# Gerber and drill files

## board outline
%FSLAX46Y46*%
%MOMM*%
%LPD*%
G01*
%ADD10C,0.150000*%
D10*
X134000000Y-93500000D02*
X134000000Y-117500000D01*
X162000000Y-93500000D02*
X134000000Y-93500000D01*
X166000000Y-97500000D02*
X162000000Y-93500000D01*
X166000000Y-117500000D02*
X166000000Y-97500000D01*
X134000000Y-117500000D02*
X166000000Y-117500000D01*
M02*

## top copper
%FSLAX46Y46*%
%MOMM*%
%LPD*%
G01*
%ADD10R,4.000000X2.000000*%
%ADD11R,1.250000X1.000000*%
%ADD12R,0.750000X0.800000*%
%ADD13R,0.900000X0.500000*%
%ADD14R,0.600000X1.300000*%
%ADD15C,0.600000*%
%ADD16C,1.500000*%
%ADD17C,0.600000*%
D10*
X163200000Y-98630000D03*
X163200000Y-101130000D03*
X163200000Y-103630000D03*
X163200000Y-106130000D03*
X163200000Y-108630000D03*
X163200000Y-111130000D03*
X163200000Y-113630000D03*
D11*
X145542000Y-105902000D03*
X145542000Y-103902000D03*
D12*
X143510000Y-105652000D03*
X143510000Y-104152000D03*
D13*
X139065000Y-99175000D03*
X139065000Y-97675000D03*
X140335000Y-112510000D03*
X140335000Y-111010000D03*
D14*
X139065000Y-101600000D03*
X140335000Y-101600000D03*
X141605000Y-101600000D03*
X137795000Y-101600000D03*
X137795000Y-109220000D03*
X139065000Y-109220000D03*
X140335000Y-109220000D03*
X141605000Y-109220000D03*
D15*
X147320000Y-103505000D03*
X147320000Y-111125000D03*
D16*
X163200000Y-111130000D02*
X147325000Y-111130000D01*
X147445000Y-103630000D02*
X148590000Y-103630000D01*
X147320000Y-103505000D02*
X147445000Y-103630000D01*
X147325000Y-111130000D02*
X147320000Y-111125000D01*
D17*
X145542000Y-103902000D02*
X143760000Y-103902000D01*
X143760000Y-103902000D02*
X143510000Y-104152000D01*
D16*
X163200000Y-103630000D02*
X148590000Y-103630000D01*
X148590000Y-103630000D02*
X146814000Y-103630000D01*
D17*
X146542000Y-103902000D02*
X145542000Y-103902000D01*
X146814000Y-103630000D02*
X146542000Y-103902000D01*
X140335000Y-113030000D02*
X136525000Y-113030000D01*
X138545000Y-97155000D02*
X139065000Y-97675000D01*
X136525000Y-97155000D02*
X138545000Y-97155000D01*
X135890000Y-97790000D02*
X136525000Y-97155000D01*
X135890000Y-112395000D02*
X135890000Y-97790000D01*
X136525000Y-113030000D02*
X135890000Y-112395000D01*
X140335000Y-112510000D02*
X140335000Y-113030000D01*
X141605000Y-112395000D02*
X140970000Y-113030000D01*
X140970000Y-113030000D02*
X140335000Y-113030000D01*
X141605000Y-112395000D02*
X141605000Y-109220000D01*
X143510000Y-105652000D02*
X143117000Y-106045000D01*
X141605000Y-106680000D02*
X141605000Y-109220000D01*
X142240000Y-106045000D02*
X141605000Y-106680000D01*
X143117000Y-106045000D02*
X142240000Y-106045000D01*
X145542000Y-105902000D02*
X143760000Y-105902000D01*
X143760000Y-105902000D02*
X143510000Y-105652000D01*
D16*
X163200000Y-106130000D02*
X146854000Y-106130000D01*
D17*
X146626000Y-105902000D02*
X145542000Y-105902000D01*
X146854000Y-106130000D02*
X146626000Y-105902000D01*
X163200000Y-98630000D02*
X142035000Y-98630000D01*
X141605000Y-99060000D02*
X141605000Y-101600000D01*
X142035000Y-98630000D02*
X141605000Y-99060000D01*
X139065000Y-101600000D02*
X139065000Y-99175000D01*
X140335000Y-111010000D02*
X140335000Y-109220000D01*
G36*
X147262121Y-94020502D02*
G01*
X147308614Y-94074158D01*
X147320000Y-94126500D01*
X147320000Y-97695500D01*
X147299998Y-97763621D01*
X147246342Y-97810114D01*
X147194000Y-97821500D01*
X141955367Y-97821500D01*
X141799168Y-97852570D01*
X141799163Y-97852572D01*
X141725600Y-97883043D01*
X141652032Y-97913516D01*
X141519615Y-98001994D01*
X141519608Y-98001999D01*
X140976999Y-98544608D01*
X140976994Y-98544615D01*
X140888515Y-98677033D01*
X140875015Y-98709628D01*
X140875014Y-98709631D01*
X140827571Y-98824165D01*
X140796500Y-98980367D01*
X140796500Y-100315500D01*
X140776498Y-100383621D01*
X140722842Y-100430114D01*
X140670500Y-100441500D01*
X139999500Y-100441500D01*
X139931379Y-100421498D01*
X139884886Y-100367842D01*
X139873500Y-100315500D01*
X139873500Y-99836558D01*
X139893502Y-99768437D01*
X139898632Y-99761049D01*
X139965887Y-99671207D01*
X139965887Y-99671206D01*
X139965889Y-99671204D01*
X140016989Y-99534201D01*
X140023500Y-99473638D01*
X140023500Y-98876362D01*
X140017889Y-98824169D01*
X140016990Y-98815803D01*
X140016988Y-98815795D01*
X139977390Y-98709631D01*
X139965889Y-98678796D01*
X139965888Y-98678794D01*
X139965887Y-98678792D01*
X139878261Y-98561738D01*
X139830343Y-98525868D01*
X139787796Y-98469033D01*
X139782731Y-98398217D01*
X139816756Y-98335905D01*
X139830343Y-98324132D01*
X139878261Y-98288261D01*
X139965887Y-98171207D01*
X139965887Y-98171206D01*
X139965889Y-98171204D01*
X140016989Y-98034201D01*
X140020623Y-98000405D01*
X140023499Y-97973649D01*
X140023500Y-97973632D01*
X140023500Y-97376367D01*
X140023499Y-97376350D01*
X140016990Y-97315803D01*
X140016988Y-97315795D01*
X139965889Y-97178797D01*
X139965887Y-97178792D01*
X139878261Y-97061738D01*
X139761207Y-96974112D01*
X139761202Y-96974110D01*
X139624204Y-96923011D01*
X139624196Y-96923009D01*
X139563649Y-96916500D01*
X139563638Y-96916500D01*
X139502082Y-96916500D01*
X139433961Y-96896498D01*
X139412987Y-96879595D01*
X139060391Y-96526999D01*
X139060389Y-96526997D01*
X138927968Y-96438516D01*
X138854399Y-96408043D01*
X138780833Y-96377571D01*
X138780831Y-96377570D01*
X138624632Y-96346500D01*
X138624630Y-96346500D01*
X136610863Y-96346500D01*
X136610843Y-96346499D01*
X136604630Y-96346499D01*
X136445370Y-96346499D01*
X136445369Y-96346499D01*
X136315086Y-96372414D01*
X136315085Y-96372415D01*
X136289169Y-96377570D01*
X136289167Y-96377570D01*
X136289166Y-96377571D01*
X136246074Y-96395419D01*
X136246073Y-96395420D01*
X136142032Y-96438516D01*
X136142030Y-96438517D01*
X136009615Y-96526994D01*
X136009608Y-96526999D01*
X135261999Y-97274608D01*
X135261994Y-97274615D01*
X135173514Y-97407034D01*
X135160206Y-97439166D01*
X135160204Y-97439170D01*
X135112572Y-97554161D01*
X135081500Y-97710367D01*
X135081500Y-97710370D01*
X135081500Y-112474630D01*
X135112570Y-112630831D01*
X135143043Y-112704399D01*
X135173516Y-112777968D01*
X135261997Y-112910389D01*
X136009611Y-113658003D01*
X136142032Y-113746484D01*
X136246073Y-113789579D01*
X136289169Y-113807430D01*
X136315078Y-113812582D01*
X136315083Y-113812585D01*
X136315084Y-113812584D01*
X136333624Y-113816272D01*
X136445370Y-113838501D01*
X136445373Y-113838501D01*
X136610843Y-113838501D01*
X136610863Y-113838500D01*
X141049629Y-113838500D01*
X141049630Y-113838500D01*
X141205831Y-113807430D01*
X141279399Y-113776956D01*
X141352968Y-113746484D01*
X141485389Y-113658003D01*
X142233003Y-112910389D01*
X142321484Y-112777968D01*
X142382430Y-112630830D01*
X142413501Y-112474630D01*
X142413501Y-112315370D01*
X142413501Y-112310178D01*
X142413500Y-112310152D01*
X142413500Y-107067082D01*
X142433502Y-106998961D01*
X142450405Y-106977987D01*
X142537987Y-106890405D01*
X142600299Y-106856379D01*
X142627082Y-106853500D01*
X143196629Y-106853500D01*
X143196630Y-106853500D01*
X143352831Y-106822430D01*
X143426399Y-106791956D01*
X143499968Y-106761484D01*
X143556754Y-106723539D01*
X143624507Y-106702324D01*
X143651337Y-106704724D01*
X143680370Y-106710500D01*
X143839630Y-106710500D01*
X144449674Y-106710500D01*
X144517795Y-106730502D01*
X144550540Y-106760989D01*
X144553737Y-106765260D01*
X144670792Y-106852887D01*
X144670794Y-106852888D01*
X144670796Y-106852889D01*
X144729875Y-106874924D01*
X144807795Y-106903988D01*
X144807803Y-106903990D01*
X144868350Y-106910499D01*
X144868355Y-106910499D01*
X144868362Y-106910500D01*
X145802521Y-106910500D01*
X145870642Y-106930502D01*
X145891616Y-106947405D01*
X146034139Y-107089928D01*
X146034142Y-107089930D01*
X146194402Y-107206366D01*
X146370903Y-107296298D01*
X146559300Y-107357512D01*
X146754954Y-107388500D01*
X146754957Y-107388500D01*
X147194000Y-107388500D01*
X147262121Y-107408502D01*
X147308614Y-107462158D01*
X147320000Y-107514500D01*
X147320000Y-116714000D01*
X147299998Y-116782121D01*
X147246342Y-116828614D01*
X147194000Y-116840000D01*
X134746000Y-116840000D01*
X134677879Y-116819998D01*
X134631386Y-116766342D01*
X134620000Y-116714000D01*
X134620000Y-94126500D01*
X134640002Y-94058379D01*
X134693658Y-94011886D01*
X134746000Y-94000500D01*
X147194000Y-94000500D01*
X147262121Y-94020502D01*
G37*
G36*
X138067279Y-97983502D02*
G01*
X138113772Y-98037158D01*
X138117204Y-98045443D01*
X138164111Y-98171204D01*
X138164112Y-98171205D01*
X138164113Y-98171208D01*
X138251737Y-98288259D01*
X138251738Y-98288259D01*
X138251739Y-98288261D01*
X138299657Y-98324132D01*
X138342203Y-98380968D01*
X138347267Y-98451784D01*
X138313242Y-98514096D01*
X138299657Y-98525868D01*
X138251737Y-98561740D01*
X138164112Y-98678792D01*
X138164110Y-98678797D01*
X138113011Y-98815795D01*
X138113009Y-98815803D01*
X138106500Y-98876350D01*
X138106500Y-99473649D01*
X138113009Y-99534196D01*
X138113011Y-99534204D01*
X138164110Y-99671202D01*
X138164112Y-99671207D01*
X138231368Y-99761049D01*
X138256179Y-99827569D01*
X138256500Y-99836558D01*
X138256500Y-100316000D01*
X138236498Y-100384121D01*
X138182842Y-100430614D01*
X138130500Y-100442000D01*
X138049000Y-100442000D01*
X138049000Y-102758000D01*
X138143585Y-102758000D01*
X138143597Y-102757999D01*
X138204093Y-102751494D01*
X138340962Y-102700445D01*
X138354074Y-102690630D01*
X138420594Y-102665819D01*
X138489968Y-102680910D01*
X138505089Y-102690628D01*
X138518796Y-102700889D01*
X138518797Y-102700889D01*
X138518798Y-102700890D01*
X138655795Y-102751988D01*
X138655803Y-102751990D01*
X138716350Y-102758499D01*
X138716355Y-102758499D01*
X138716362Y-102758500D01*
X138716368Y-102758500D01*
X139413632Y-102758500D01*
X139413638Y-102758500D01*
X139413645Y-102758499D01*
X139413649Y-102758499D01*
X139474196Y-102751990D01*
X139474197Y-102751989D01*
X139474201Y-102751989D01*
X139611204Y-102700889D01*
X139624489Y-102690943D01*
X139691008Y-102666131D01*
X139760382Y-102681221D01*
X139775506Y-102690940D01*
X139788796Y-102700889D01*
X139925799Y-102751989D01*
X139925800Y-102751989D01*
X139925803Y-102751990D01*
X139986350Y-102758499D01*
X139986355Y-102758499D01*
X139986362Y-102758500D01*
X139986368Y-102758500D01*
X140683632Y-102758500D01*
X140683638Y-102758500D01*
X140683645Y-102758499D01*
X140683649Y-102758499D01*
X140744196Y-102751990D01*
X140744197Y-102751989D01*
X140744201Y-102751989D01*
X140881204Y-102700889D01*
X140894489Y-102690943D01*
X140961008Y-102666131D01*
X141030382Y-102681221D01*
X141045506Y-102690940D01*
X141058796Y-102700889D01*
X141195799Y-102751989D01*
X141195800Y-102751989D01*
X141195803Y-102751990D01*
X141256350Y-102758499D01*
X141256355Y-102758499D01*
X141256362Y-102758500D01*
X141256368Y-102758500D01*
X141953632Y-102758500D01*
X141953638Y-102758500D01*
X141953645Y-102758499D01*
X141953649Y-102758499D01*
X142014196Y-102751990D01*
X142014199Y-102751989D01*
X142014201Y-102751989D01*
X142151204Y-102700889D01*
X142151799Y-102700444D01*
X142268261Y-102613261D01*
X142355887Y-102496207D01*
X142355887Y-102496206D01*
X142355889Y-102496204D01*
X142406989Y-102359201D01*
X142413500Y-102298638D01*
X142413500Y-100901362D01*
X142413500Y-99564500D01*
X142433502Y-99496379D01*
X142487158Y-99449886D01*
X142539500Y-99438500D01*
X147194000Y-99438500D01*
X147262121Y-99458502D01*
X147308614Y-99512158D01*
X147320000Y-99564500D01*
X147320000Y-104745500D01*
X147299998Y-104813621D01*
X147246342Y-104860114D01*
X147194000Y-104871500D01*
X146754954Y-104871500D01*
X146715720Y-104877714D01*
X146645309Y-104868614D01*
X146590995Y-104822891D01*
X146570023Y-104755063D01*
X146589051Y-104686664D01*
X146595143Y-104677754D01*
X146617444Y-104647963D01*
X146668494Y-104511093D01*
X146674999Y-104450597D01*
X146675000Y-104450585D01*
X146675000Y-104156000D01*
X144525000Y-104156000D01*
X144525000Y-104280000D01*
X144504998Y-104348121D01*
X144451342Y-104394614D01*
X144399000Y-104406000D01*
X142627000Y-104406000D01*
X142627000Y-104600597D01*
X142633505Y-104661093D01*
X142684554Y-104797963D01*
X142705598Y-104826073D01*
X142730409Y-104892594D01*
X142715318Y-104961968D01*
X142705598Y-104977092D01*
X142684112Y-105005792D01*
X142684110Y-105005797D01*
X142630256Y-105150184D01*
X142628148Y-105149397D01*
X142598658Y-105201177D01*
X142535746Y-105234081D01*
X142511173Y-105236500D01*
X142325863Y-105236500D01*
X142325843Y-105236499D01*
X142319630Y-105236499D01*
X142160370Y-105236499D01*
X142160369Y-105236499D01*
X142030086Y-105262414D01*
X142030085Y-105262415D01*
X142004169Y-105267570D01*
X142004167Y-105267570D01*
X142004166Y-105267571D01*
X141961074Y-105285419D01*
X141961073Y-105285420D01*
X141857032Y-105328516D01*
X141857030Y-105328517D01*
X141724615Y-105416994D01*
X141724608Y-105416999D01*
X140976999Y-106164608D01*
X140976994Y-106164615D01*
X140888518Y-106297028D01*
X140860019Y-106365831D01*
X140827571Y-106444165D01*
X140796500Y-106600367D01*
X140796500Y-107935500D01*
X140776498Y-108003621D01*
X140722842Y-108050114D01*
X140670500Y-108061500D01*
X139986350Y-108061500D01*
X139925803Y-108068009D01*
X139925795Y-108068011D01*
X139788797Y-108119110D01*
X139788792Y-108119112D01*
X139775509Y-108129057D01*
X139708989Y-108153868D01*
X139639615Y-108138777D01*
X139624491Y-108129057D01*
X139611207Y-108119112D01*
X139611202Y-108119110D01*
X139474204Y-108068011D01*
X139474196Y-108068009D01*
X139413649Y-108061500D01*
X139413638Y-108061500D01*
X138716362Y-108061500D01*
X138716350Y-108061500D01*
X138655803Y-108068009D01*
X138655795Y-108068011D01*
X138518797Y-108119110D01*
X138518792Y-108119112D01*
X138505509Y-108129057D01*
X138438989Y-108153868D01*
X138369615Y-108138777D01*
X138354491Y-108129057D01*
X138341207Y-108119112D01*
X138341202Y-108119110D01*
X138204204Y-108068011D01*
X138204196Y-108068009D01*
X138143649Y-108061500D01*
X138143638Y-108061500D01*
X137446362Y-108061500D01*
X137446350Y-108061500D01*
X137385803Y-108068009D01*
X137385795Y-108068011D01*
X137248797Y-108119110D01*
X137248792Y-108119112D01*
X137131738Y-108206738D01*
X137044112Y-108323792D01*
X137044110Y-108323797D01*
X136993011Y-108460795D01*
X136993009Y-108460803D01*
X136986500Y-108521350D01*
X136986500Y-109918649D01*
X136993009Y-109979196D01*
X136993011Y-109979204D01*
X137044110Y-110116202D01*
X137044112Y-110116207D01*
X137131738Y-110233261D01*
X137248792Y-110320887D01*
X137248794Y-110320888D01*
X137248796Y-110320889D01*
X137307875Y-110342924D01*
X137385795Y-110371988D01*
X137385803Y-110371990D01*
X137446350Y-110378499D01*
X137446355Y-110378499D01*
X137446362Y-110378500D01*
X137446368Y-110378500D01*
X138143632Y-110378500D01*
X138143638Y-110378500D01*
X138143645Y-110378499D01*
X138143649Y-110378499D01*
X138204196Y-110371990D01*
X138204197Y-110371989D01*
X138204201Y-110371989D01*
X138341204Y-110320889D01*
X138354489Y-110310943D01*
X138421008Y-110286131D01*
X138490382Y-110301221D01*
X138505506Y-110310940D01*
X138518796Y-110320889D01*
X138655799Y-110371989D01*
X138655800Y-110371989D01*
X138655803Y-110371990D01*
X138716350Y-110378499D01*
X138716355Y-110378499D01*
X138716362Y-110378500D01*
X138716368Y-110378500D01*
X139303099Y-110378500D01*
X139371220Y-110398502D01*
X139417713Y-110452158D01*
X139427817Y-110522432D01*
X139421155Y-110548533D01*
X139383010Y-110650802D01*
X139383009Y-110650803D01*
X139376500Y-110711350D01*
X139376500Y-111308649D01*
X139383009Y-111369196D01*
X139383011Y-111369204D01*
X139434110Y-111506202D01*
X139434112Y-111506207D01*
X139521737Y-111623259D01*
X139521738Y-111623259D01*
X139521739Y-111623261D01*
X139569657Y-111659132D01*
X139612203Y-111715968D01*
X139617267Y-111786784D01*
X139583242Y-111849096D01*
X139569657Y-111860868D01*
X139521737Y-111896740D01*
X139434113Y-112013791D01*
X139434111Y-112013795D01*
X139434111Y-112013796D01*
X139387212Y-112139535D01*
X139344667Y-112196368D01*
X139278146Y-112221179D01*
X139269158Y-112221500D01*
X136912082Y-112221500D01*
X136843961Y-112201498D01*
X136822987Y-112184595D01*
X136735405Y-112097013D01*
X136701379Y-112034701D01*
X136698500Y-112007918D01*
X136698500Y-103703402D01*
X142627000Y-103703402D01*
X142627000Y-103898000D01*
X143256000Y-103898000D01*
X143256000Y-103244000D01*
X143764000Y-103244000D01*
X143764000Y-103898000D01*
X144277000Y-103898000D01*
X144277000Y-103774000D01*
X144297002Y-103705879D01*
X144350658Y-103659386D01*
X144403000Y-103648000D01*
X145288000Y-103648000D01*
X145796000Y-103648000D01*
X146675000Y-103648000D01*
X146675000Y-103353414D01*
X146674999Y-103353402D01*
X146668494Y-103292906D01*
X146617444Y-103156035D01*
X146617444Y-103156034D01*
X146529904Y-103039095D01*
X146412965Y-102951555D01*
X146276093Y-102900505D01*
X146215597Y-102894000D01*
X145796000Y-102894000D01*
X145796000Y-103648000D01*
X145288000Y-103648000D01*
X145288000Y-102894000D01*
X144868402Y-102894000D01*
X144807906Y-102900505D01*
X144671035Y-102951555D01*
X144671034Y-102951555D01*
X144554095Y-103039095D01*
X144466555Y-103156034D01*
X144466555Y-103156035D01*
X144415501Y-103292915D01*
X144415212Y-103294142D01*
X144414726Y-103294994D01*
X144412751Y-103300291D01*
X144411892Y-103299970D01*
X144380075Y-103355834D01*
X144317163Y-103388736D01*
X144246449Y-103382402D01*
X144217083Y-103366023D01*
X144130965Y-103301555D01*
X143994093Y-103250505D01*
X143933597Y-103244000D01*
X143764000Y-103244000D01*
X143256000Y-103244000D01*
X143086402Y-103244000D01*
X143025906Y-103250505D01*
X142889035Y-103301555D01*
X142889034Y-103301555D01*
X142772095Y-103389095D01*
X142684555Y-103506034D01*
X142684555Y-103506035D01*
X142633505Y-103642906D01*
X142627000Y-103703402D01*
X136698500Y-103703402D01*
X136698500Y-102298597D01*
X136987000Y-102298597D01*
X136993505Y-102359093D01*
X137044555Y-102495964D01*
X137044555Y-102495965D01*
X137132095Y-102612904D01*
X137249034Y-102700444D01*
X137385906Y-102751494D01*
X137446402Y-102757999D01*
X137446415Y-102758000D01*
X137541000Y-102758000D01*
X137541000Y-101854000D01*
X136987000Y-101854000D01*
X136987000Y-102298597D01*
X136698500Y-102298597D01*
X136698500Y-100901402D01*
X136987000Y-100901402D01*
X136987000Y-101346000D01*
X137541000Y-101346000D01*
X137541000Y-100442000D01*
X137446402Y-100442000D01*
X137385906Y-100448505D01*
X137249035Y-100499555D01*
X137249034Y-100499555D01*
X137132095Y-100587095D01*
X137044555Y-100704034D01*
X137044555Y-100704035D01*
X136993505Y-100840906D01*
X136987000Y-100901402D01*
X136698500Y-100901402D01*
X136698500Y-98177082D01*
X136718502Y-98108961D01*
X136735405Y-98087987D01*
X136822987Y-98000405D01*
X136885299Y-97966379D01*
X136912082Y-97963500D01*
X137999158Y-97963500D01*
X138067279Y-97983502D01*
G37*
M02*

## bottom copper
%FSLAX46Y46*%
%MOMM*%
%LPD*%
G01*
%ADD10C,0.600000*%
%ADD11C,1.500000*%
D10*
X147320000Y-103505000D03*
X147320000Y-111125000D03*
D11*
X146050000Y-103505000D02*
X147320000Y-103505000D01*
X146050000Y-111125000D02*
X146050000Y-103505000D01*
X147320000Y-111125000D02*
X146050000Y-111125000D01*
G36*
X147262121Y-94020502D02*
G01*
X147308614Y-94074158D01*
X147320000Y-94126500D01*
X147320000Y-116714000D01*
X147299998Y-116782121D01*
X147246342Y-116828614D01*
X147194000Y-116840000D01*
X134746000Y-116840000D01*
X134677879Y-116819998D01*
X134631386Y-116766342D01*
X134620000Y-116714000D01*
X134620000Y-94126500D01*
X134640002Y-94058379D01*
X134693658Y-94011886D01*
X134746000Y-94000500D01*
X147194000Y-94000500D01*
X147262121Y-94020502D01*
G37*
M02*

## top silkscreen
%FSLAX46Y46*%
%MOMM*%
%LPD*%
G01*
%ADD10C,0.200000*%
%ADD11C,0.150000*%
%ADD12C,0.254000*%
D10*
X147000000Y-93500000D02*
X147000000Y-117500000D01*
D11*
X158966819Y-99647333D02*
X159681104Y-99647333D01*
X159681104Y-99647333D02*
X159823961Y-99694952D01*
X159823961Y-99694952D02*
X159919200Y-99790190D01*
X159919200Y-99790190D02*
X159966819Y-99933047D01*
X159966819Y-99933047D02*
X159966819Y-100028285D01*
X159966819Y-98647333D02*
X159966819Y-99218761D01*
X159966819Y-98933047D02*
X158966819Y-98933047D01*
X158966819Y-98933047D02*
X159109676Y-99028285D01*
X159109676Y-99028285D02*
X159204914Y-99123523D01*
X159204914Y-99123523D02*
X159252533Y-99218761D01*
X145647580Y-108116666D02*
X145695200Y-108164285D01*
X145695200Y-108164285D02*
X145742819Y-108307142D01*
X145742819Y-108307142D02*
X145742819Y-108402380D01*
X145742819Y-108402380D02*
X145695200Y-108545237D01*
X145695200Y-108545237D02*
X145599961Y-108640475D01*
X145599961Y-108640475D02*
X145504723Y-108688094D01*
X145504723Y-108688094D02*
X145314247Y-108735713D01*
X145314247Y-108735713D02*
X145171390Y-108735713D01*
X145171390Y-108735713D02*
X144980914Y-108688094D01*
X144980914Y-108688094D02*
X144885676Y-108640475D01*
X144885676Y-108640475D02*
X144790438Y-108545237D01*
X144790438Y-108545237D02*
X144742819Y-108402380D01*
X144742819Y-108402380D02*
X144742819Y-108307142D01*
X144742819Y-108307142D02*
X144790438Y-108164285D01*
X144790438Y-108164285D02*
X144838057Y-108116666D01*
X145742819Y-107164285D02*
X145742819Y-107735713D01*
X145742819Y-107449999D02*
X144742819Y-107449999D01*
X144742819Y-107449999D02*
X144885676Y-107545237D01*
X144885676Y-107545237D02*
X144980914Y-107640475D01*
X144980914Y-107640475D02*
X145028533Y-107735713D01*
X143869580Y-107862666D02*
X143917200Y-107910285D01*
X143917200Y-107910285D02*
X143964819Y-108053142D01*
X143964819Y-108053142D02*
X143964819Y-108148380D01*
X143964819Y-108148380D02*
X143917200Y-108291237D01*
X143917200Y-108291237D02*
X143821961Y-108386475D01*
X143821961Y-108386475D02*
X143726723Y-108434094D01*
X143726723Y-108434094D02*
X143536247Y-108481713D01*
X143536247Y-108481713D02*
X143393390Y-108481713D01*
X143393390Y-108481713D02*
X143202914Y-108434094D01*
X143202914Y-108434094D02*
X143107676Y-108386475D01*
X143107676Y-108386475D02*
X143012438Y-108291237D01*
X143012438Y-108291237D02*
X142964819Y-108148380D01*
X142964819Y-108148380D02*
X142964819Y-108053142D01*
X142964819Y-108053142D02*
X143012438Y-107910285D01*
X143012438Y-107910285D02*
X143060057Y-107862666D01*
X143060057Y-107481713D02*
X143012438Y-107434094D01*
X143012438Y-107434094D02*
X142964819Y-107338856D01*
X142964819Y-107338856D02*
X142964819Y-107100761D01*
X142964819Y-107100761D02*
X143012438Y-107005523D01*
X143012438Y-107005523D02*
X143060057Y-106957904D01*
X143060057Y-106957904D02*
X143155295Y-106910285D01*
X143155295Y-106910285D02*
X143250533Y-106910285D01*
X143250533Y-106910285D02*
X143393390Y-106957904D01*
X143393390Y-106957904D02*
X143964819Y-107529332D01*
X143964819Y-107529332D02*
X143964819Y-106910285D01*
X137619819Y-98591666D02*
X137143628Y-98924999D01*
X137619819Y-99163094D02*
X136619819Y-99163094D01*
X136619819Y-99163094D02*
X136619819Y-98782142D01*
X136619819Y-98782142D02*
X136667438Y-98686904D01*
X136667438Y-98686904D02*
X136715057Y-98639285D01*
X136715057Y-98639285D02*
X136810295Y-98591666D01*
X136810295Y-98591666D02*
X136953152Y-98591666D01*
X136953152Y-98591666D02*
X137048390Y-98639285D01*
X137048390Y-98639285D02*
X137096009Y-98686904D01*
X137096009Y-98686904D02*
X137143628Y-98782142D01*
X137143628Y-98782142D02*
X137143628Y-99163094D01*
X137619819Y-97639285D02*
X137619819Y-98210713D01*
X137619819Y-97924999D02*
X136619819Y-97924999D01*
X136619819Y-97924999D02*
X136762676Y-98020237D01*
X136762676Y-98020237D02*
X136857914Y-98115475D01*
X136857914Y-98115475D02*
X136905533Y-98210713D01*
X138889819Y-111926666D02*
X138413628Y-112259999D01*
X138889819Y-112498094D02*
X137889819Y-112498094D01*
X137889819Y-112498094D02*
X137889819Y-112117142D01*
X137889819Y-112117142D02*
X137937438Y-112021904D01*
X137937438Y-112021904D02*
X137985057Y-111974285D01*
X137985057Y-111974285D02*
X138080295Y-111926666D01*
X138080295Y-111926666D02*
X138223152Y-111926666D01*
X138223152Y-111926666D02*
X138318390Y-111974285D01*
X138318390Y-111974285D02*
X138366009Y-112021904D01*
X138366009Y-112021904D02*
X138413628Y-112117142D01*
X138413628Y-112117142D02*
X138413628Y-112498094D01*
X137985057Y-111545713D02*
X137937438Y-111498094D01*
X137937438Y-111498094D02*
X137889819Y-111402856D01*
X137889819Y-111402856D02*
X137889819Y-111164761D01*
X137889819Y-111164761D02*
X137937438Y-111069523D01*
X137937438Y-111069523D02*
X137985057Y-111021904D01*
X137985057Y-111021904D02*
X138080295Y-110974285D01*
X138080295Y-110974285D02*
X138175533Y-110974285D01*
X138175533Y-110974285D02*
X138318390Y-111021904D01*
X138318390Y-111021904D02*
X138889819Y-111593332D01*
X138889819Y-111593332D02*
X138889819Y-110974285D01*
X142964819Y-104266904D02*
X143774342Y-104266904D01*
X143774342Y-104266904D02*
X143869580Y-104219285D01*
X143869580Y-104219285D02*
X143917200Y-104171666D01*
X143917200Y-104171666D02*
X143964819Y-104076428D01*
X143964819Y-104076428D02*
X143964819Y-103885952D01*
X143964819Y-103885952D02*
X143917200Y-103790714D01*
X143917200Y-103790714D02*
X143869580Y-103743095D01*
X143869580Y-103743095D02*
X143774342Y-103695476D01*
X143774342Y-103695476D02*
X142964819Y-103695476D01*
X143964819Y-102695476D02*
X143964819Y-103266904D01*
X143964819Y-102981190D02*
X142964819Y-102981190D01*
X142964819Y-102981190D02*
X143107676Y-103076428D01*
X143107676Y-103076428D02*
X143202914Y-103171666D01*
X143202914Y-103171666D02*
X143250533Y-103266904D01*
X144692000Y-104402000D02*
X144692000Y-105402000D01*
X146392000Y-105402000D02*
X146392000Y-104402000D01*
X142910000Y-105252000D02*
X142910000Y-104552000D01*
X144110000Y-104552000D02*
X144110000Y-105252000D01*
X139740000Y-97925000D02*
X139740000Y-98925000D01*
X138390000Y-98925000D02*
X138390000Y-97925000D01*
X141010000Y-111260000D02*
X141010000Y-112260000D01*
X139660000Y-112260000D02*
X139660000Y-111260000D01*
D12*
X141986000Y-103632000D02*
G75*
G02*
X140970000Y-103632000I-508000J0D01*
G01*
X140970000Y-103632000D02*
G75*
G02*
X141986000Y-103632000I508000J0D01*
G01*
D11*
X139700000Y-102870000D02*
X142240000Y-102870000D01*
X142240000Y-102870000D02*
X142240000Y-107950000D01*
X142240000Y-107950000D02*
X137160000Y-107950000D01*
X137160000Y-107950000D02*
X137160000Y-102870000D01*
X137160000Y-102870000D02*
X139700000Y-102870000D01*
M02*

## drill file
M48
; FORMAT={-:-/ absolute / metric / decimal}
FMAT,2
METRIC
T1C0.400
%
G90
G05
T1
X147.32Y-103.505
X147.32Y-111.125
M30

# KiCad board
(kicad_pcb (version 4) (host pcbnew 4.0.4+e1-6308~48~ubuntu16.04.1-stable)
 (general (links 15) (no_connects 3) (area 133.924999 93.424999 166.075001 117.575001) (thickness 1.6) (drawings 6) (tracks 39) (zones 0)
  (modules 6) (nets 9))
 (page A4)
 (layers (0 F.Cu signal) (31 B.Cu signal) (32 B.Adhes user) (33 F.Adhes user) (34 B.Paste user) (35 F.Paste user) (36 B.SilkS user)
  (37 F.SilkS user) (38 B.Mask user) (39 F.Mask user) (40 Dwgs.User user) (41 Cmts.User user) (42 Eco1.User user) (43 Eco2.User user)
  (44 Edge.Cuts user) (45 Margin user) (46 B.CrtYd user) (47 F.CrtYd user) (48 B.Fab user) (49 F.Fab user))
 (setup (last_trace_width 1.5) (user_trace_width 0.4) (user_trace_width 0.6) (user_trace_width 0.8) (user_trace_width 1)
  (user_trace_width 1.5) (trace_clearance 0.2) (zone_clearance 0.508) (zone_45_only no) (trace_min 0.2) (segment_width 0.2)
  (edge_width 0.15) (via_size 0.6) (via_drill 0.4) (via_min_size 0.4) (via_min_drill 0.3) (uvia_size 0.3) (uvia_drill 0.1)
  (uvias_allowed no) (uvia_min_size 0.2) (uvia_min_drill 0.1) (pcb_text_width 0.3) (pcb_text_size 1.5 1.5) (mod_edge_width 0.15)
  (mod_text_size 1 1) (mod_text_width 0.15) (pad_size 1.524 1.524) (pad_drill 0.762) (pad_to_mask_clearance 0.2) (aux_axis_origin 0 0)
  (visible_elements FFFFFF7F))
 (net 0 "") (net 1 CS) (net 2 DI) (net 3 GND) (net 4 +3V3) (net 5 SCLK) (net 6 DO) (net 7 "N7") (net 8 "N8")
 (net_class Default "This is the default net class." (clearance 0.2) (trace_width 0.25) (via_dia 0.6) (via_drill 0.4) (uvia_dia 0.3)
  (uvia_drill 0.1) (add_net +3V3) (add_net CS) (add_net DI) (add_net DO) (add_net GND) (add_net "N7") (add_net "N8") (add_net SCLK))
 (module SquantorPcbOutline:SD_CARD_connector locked (layer F.Cu) (at 163.2 106.13)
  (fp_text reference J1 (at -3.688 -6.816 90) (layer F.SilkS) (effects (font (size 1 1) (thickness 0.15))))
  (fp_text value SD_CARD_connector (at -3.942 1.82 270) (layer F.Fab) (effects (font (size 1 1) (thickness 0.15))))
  (pad 1 smd rect (at 0 -7.5 90) (size 2 4) (layers F.Cu F.Paste F.Mask) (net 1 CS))
  (pad 2 smd rect (at 0 -5 90) (size 2 4) (layers F.Cu F.Paste F.Mask) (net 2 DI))
  (pad 3 smd rect (at 0 -2.5 90) (size 2 4) (layers F.Cu F.Paste F.Mask) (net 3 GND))
  (pad 4 smd rect (at 0 0 90) (size 2 4) (layers F.Cu F.Paste F.Mask) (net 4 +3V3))
  (pad 5 smd rect (at 0 2.5 90) (size 2 4) (layers F.Cu F.Paste F.Mask) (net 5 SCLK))
  (pad 6 smd rect (at 0 5 90) (size 2 4) (layers F.Cu F.Paste F.Mask) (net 3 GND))
  (pad 7 smd rect (at 0 7.5 90) (size 2 4) (layers F.Cu F.Paste F.Mask) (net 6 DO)))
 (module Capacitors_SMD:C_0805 (layer F.Cu) (at 145.542 104.902 90)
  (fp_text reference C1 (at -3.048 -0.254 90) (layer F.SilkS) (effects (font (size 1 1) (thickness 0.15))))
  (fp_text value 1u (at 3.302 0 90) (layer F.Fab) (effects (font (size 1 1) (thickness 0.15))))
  (fp_line (start 0.5 -0.85) (end -0.5 -0.85) (layer F.SilkS) (width 0.15))
  (fp_line (start -0.5 0.85) (end 0.5 0.85) (layer F.SilkS) (width 0.15))
  (pad 1 smd rect (at -1 0 90) (size 1 1.25) (layers F.Cu F.Paste F.Mask) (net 4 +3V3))
  (pad 2 smd rect (at 1 0 90) (size 1 1.25) (layers F.Cu F.Paste F.Mask) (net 3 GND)))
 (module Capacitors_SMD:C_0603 (layer F.Cu) (at 143.51 104.902 90)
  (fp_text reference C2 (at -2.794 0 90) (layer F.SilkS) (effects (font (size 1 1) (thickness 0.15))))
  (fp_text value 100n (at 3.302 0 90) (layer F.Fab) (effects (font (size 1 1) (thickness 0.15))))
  (fp_line (start -0.35 -0.6) (end 0.35 -0.6) (layer F.SilkS) (width 0.15))
  (fp_line (start 0.35 0.6) (end -0.35 0.6) (layer F.SilkS) (width 0.15))
  (pad 1 smd rect (at -0.75 0 90) (size 0.8 0.75) (layers F.Cu F.Paste F.Mask) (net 4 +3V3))
  (pad 2 smd rect (at 0.75 0 90) (size 0.8 0.75) (layers F.Cu F.Paste F.Mask) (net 3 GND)))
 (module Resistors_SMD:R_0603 (layer F.Cu) (at 139.065 98.425 90)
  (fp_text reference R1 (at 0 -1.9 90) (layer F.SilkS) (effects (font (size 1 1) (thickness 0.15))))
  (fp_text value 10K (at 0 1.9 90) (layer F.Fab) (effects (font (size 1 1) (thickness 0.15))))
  (fp_line (start 0.5 0.675) (end -0.5 0.675) (layer F.SilkS) (width 0.15))
  (fp_line (start -0.5 -0.675) (end 0.5 -0.675) (layer F.SilkS) (width 0.15))
  (pad 1 smd rect (at -0.75 0 90) (size 0.5 0.9) (layers F.Cu F.Paste F.Mask) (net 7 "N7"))
  (pad 2 smd rect (at 0.75 0 90) (size 0.5 0.9) (layers F.Cu F.Paste F.Mask) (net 4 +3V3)))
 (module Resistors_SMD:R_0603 (layer F.Cu) (at 140.335 111.76 90)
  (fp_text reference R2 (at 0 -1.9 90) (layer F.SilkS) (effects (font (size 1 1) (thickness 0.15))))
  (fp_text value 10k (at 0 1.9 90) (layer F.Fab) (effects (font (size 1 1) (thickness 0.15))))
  (fp_line (start 0.5 0.675) (end -0.5 0.675) (layer F.SilkS) (width 0.15))
  (fp_line (start -0.5 -0.675) (end 0.5 -0.675) (layer F.SilkS) (width 0.15))
  (pad 1 smd rect (at -0.75 0 90) (size 0.5 0.9) (layers F.Cu F.Paste F.Mask) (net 4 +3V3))
  (pad 2 smd rect (at 0.75 0 90) (size 0.5 0.9) (layers F.Cu F.Paste F.Mask) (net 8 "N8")))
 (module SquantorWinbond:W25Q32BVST (layer F.Cu) (at 139.7 105.41 270)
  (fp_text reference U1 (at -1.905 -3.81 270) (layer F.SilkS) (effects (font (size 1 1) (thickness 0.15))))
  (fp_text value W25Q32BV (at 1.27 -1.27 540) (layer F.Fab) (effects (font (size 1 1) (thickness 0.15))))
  (fp_circle (center -1.778 -1.778) (end -1.27 -1.778) (layer F.SilkS) (width 0.254))
  (fp_line (start -2.54 0) (end -2.54 -2.54) (layer F.SilkS) (width 0.15))
  (fp_line (start -2.54 -2.54) (end 2.54 -2.54) (layer F.SilkS) (width 0.15))
  (fp_line (start 2.54 -2.54) (end 2.54 2.54) (layer F.SilkS) (width 0.15))
  (fp_line (start 2.54 2.54) (end -2.54 2.54) (layer F.SilkS) (width 0.15))
  (fp_line (start -2.54 2.54) (end -2.54 0) (layer F.SilkS) (width 0.15))
  (pad 3 smd rect (at -3.81 0.635 270) (size 1.3 0.6) (layers F.Cu F.Paste F.Mask) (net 7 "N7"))
  (pad 2 smd rect (at -3.81 -0.635 270) (size 1.3 0.6) (layers F.Cu F.Paste F.Mask) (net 6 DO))
  (pad 1 smd rect (at -3.81 -1.905 270) (size 1.3 0.6) (layers F.Cu F.Paste F.Mask) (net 1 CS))
  (pad 4 smd rect (at -3.81 1.905 270) (size 1.3 0.6) (layers F.Cu F.Paste F.Mask) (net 3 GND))
  (pad 5 smd rect (at 3.81 1.905 270) (size 1.3 0.6) (layers F.Cu F.Paste F.Mask) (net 2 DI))
  (pad 6 smd rect (at 3.81 0.635 270) (size 1.3 0.6) (layers F.Cu F.Paste F.Mask) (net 5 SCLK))
  (pad 7 smd rect (at 3.81 -0.635 270) (size 1.3 0.6) (layers F.Cu F.Paste F.Mask) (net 8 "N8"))
  (pad 8 smd rect (at 3.81 -1.905 270) (size 1.3 0.6) (layers F.Cu F.Paste F.Mask) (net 4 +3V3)))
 (gr_line (start 147 93.5) (end 147 117.5) (angle 90) (layer F.SilkS) (width 0.2))
 (gr_line (start 134 93.5) (end 134 117.5) (angle 90) (layer Edge.Cuts) (width 0.15))
 (gr_line (start 162 93.5) (end 134 93.5) (angle 90) (layer Edge.Cuts) (width 0.15))
 (gr_line (start 166 97.5) (end 162 93.5) (angle 90) (layer Edge.Cuts) (width 0.15))
 (gr_line (start 166 117.5) (end 166 97.5) (angle 90) (layer Edge.Cuts) (width 0.15))
 (gr_line (start 134 117.5) (end 166 117.5) (angle 90) (layer Edge.Cuts) (width 0.15))
 (segment (start 163.2 111.13) (end 147.325 111.13) (width 1.5) (layer F.Cu) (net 3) (status 400000))
 (segment (start 147.445 103.63) (end 148.59 103.63) (width 1.5) (layer F.Cu) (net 3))
 (segment (start 147.32 103.505) (end 147.445 103.63) (width 1.5) (layer F.Cu) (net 3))
 (via (at 147.32 103.505) (size 0.6) (drill 0.4) (layers F.Cu B.Cu) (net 3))
 (segment (start 146.05 103.505) (end 147.32 103.505) (width 1.5) (layer B.Cu) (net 3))
 (segment (start 146.05 111.125) (end 146.05 103.505) (width 1.5) (layer B.Cu) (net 3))
 (segment (start 147.32 111.125) (end 146.05 111.125) (width 1.5) (layer B.Cu) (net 3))
 (via (at 147.32 111.125) (size 0.6) (drill 0.4) (layers F.Cu B.Cu) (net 3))
 (segment (start 147.325 111.13) (end 147.32 111.125) (width 1.5) (layer F.Cu) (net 3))
 (segment (start 145.542 103.902) (end 143.76 103.902) (width 0.6) (layer F.Cu) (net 3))
 (segment (start 143.76 103.902) (end 143.51 104.152) (width 0.6) (layer F.Cu) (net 3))
 (segment (start 163.2 103.63) (end 148.59 103.63) (width 1.5) (layer F.Cu) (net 3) (status 10))
 (segment (start 148.59 103.63) (end 146.814 103.63) (width 1.5) (layer F.Cu) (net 3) (status 10))
 (segment (start 146.542 103.902) (end 145.542 103.902) (width 0.6) (layer F.Cu) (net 3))
 (segment (start 146.814 103.63) (end 146.542 103.902) (width 0.6) (layer F.Cu) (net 3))
 (segment (start 140.335 113.03) (end 136.525 113.03) (width 0.6) (layer F.Cu) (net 4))
 (segment (start 138.545 97.155) (end 139.065 97.675) (width 0.6) (layer F.Cu) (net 4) (status 800000))
 (segment (start 136.525 97.155) (end 138.545 97.155) (width 0.6) (layer F.Cu) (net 4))
 (segment (start 135.89 97.79) (end 136.525 97.155) (width 0.6) (layer F.Cu) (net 4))
 (segment (start 135.89 112.395) (end 135.89 97.79) (width 0.6) (layer F.Cu) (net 4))
 (segment (start 136.525 113.03) (end 135.89 112.395) (width 0.6) (layer F.Cu) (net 4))
 (segment (start 140.335 112.51) (end 140.335 113.03) (width 0.6) (layer F.Cu) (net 4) (status 400010))
 (segment (start 141.605 112.395) (end 140.97 113.03) (width 0.6) (layer F.Cu) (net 4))
 (segment (start 140.97 113.03) (end 140.335 113.03) (width 0.6) (layer F.Cu) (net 4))
 (segment (start 141.605 112.395) (end 141.605 109.22) (width 0.6) (layer F.Cu) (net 4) (status 800000))
 (segment (start 143.51 105.652) (end 143.117 106.045) (width 0.6) (layer F.Cu) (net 4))
 (segment (start 141.605 106.68) (end 141.605 109.22) (width 0.6) (layer F.Cu) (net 4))
 (segment (start 142.24 106.045) (end 141.605 106.68) (width 0.6) (layer F.Cu) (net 4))
 (segment (start 143.117 106.045) (end 142.24 106.045) (width 0.6) (layer F.Cu) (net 4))
 (segment (start 145.542 105.902) (end 143.76 105.902) (width 0.6) (layer F.Cu) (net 4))
 (segment (start 143.76 105.902) (end 143.51 105.652) (width 0.6) (layer F.Cu) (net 4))
 (segment (start 163.2 106.13) (end 146.854 106.13) (width 1.5) (layer F.Cu) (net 4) (status 10))
 (segment (start 146.626 105.902) (end 145.542 105.902) (width 0.6) (layer F.Cu) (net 4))
 (segment (start 146.854 106.13) (end 146.626 105.902) (width 0.6) (layer F.Cu) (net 4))
 (segment (start 163.2 98.63) (end 142.035 98.63) (width 0.6) (layer F.Cu) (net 1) (status 400000))
 (segment (start 141.605 99.06) (end 141.605 101.6) (width 0.6) (layer F.Cu) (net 1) (status 800000))
 (segment (start 142.035 98.63) (end 141.605 99.06) (width 0.6) (layer F.Cu) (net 1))
 (segment (start 139.065 101.6) (end 139.065 99.175) (width 0.6) (layer F.Cu) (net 7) (status C00000))
 (segment (start 140.335 111.01) (end 140.335 109.22) (width 0.6) (layer F.Cu) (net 8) (status 10))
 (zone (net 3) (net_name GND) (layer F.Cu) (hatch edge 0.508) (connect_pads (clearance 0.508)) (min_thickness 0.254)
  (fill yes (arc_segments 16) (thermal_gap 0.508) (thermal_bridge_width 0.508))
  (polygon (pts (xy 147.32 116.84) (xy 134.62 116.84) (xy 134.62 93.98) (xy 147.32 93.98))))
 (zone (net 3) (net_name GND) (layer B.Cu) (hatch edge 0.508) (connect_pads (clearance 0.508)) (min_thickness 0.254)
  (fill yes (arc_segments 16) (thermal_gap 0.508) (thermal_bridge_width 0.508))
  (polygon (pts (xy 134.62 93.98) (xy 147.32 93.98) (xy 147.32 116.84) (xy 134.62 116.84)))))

